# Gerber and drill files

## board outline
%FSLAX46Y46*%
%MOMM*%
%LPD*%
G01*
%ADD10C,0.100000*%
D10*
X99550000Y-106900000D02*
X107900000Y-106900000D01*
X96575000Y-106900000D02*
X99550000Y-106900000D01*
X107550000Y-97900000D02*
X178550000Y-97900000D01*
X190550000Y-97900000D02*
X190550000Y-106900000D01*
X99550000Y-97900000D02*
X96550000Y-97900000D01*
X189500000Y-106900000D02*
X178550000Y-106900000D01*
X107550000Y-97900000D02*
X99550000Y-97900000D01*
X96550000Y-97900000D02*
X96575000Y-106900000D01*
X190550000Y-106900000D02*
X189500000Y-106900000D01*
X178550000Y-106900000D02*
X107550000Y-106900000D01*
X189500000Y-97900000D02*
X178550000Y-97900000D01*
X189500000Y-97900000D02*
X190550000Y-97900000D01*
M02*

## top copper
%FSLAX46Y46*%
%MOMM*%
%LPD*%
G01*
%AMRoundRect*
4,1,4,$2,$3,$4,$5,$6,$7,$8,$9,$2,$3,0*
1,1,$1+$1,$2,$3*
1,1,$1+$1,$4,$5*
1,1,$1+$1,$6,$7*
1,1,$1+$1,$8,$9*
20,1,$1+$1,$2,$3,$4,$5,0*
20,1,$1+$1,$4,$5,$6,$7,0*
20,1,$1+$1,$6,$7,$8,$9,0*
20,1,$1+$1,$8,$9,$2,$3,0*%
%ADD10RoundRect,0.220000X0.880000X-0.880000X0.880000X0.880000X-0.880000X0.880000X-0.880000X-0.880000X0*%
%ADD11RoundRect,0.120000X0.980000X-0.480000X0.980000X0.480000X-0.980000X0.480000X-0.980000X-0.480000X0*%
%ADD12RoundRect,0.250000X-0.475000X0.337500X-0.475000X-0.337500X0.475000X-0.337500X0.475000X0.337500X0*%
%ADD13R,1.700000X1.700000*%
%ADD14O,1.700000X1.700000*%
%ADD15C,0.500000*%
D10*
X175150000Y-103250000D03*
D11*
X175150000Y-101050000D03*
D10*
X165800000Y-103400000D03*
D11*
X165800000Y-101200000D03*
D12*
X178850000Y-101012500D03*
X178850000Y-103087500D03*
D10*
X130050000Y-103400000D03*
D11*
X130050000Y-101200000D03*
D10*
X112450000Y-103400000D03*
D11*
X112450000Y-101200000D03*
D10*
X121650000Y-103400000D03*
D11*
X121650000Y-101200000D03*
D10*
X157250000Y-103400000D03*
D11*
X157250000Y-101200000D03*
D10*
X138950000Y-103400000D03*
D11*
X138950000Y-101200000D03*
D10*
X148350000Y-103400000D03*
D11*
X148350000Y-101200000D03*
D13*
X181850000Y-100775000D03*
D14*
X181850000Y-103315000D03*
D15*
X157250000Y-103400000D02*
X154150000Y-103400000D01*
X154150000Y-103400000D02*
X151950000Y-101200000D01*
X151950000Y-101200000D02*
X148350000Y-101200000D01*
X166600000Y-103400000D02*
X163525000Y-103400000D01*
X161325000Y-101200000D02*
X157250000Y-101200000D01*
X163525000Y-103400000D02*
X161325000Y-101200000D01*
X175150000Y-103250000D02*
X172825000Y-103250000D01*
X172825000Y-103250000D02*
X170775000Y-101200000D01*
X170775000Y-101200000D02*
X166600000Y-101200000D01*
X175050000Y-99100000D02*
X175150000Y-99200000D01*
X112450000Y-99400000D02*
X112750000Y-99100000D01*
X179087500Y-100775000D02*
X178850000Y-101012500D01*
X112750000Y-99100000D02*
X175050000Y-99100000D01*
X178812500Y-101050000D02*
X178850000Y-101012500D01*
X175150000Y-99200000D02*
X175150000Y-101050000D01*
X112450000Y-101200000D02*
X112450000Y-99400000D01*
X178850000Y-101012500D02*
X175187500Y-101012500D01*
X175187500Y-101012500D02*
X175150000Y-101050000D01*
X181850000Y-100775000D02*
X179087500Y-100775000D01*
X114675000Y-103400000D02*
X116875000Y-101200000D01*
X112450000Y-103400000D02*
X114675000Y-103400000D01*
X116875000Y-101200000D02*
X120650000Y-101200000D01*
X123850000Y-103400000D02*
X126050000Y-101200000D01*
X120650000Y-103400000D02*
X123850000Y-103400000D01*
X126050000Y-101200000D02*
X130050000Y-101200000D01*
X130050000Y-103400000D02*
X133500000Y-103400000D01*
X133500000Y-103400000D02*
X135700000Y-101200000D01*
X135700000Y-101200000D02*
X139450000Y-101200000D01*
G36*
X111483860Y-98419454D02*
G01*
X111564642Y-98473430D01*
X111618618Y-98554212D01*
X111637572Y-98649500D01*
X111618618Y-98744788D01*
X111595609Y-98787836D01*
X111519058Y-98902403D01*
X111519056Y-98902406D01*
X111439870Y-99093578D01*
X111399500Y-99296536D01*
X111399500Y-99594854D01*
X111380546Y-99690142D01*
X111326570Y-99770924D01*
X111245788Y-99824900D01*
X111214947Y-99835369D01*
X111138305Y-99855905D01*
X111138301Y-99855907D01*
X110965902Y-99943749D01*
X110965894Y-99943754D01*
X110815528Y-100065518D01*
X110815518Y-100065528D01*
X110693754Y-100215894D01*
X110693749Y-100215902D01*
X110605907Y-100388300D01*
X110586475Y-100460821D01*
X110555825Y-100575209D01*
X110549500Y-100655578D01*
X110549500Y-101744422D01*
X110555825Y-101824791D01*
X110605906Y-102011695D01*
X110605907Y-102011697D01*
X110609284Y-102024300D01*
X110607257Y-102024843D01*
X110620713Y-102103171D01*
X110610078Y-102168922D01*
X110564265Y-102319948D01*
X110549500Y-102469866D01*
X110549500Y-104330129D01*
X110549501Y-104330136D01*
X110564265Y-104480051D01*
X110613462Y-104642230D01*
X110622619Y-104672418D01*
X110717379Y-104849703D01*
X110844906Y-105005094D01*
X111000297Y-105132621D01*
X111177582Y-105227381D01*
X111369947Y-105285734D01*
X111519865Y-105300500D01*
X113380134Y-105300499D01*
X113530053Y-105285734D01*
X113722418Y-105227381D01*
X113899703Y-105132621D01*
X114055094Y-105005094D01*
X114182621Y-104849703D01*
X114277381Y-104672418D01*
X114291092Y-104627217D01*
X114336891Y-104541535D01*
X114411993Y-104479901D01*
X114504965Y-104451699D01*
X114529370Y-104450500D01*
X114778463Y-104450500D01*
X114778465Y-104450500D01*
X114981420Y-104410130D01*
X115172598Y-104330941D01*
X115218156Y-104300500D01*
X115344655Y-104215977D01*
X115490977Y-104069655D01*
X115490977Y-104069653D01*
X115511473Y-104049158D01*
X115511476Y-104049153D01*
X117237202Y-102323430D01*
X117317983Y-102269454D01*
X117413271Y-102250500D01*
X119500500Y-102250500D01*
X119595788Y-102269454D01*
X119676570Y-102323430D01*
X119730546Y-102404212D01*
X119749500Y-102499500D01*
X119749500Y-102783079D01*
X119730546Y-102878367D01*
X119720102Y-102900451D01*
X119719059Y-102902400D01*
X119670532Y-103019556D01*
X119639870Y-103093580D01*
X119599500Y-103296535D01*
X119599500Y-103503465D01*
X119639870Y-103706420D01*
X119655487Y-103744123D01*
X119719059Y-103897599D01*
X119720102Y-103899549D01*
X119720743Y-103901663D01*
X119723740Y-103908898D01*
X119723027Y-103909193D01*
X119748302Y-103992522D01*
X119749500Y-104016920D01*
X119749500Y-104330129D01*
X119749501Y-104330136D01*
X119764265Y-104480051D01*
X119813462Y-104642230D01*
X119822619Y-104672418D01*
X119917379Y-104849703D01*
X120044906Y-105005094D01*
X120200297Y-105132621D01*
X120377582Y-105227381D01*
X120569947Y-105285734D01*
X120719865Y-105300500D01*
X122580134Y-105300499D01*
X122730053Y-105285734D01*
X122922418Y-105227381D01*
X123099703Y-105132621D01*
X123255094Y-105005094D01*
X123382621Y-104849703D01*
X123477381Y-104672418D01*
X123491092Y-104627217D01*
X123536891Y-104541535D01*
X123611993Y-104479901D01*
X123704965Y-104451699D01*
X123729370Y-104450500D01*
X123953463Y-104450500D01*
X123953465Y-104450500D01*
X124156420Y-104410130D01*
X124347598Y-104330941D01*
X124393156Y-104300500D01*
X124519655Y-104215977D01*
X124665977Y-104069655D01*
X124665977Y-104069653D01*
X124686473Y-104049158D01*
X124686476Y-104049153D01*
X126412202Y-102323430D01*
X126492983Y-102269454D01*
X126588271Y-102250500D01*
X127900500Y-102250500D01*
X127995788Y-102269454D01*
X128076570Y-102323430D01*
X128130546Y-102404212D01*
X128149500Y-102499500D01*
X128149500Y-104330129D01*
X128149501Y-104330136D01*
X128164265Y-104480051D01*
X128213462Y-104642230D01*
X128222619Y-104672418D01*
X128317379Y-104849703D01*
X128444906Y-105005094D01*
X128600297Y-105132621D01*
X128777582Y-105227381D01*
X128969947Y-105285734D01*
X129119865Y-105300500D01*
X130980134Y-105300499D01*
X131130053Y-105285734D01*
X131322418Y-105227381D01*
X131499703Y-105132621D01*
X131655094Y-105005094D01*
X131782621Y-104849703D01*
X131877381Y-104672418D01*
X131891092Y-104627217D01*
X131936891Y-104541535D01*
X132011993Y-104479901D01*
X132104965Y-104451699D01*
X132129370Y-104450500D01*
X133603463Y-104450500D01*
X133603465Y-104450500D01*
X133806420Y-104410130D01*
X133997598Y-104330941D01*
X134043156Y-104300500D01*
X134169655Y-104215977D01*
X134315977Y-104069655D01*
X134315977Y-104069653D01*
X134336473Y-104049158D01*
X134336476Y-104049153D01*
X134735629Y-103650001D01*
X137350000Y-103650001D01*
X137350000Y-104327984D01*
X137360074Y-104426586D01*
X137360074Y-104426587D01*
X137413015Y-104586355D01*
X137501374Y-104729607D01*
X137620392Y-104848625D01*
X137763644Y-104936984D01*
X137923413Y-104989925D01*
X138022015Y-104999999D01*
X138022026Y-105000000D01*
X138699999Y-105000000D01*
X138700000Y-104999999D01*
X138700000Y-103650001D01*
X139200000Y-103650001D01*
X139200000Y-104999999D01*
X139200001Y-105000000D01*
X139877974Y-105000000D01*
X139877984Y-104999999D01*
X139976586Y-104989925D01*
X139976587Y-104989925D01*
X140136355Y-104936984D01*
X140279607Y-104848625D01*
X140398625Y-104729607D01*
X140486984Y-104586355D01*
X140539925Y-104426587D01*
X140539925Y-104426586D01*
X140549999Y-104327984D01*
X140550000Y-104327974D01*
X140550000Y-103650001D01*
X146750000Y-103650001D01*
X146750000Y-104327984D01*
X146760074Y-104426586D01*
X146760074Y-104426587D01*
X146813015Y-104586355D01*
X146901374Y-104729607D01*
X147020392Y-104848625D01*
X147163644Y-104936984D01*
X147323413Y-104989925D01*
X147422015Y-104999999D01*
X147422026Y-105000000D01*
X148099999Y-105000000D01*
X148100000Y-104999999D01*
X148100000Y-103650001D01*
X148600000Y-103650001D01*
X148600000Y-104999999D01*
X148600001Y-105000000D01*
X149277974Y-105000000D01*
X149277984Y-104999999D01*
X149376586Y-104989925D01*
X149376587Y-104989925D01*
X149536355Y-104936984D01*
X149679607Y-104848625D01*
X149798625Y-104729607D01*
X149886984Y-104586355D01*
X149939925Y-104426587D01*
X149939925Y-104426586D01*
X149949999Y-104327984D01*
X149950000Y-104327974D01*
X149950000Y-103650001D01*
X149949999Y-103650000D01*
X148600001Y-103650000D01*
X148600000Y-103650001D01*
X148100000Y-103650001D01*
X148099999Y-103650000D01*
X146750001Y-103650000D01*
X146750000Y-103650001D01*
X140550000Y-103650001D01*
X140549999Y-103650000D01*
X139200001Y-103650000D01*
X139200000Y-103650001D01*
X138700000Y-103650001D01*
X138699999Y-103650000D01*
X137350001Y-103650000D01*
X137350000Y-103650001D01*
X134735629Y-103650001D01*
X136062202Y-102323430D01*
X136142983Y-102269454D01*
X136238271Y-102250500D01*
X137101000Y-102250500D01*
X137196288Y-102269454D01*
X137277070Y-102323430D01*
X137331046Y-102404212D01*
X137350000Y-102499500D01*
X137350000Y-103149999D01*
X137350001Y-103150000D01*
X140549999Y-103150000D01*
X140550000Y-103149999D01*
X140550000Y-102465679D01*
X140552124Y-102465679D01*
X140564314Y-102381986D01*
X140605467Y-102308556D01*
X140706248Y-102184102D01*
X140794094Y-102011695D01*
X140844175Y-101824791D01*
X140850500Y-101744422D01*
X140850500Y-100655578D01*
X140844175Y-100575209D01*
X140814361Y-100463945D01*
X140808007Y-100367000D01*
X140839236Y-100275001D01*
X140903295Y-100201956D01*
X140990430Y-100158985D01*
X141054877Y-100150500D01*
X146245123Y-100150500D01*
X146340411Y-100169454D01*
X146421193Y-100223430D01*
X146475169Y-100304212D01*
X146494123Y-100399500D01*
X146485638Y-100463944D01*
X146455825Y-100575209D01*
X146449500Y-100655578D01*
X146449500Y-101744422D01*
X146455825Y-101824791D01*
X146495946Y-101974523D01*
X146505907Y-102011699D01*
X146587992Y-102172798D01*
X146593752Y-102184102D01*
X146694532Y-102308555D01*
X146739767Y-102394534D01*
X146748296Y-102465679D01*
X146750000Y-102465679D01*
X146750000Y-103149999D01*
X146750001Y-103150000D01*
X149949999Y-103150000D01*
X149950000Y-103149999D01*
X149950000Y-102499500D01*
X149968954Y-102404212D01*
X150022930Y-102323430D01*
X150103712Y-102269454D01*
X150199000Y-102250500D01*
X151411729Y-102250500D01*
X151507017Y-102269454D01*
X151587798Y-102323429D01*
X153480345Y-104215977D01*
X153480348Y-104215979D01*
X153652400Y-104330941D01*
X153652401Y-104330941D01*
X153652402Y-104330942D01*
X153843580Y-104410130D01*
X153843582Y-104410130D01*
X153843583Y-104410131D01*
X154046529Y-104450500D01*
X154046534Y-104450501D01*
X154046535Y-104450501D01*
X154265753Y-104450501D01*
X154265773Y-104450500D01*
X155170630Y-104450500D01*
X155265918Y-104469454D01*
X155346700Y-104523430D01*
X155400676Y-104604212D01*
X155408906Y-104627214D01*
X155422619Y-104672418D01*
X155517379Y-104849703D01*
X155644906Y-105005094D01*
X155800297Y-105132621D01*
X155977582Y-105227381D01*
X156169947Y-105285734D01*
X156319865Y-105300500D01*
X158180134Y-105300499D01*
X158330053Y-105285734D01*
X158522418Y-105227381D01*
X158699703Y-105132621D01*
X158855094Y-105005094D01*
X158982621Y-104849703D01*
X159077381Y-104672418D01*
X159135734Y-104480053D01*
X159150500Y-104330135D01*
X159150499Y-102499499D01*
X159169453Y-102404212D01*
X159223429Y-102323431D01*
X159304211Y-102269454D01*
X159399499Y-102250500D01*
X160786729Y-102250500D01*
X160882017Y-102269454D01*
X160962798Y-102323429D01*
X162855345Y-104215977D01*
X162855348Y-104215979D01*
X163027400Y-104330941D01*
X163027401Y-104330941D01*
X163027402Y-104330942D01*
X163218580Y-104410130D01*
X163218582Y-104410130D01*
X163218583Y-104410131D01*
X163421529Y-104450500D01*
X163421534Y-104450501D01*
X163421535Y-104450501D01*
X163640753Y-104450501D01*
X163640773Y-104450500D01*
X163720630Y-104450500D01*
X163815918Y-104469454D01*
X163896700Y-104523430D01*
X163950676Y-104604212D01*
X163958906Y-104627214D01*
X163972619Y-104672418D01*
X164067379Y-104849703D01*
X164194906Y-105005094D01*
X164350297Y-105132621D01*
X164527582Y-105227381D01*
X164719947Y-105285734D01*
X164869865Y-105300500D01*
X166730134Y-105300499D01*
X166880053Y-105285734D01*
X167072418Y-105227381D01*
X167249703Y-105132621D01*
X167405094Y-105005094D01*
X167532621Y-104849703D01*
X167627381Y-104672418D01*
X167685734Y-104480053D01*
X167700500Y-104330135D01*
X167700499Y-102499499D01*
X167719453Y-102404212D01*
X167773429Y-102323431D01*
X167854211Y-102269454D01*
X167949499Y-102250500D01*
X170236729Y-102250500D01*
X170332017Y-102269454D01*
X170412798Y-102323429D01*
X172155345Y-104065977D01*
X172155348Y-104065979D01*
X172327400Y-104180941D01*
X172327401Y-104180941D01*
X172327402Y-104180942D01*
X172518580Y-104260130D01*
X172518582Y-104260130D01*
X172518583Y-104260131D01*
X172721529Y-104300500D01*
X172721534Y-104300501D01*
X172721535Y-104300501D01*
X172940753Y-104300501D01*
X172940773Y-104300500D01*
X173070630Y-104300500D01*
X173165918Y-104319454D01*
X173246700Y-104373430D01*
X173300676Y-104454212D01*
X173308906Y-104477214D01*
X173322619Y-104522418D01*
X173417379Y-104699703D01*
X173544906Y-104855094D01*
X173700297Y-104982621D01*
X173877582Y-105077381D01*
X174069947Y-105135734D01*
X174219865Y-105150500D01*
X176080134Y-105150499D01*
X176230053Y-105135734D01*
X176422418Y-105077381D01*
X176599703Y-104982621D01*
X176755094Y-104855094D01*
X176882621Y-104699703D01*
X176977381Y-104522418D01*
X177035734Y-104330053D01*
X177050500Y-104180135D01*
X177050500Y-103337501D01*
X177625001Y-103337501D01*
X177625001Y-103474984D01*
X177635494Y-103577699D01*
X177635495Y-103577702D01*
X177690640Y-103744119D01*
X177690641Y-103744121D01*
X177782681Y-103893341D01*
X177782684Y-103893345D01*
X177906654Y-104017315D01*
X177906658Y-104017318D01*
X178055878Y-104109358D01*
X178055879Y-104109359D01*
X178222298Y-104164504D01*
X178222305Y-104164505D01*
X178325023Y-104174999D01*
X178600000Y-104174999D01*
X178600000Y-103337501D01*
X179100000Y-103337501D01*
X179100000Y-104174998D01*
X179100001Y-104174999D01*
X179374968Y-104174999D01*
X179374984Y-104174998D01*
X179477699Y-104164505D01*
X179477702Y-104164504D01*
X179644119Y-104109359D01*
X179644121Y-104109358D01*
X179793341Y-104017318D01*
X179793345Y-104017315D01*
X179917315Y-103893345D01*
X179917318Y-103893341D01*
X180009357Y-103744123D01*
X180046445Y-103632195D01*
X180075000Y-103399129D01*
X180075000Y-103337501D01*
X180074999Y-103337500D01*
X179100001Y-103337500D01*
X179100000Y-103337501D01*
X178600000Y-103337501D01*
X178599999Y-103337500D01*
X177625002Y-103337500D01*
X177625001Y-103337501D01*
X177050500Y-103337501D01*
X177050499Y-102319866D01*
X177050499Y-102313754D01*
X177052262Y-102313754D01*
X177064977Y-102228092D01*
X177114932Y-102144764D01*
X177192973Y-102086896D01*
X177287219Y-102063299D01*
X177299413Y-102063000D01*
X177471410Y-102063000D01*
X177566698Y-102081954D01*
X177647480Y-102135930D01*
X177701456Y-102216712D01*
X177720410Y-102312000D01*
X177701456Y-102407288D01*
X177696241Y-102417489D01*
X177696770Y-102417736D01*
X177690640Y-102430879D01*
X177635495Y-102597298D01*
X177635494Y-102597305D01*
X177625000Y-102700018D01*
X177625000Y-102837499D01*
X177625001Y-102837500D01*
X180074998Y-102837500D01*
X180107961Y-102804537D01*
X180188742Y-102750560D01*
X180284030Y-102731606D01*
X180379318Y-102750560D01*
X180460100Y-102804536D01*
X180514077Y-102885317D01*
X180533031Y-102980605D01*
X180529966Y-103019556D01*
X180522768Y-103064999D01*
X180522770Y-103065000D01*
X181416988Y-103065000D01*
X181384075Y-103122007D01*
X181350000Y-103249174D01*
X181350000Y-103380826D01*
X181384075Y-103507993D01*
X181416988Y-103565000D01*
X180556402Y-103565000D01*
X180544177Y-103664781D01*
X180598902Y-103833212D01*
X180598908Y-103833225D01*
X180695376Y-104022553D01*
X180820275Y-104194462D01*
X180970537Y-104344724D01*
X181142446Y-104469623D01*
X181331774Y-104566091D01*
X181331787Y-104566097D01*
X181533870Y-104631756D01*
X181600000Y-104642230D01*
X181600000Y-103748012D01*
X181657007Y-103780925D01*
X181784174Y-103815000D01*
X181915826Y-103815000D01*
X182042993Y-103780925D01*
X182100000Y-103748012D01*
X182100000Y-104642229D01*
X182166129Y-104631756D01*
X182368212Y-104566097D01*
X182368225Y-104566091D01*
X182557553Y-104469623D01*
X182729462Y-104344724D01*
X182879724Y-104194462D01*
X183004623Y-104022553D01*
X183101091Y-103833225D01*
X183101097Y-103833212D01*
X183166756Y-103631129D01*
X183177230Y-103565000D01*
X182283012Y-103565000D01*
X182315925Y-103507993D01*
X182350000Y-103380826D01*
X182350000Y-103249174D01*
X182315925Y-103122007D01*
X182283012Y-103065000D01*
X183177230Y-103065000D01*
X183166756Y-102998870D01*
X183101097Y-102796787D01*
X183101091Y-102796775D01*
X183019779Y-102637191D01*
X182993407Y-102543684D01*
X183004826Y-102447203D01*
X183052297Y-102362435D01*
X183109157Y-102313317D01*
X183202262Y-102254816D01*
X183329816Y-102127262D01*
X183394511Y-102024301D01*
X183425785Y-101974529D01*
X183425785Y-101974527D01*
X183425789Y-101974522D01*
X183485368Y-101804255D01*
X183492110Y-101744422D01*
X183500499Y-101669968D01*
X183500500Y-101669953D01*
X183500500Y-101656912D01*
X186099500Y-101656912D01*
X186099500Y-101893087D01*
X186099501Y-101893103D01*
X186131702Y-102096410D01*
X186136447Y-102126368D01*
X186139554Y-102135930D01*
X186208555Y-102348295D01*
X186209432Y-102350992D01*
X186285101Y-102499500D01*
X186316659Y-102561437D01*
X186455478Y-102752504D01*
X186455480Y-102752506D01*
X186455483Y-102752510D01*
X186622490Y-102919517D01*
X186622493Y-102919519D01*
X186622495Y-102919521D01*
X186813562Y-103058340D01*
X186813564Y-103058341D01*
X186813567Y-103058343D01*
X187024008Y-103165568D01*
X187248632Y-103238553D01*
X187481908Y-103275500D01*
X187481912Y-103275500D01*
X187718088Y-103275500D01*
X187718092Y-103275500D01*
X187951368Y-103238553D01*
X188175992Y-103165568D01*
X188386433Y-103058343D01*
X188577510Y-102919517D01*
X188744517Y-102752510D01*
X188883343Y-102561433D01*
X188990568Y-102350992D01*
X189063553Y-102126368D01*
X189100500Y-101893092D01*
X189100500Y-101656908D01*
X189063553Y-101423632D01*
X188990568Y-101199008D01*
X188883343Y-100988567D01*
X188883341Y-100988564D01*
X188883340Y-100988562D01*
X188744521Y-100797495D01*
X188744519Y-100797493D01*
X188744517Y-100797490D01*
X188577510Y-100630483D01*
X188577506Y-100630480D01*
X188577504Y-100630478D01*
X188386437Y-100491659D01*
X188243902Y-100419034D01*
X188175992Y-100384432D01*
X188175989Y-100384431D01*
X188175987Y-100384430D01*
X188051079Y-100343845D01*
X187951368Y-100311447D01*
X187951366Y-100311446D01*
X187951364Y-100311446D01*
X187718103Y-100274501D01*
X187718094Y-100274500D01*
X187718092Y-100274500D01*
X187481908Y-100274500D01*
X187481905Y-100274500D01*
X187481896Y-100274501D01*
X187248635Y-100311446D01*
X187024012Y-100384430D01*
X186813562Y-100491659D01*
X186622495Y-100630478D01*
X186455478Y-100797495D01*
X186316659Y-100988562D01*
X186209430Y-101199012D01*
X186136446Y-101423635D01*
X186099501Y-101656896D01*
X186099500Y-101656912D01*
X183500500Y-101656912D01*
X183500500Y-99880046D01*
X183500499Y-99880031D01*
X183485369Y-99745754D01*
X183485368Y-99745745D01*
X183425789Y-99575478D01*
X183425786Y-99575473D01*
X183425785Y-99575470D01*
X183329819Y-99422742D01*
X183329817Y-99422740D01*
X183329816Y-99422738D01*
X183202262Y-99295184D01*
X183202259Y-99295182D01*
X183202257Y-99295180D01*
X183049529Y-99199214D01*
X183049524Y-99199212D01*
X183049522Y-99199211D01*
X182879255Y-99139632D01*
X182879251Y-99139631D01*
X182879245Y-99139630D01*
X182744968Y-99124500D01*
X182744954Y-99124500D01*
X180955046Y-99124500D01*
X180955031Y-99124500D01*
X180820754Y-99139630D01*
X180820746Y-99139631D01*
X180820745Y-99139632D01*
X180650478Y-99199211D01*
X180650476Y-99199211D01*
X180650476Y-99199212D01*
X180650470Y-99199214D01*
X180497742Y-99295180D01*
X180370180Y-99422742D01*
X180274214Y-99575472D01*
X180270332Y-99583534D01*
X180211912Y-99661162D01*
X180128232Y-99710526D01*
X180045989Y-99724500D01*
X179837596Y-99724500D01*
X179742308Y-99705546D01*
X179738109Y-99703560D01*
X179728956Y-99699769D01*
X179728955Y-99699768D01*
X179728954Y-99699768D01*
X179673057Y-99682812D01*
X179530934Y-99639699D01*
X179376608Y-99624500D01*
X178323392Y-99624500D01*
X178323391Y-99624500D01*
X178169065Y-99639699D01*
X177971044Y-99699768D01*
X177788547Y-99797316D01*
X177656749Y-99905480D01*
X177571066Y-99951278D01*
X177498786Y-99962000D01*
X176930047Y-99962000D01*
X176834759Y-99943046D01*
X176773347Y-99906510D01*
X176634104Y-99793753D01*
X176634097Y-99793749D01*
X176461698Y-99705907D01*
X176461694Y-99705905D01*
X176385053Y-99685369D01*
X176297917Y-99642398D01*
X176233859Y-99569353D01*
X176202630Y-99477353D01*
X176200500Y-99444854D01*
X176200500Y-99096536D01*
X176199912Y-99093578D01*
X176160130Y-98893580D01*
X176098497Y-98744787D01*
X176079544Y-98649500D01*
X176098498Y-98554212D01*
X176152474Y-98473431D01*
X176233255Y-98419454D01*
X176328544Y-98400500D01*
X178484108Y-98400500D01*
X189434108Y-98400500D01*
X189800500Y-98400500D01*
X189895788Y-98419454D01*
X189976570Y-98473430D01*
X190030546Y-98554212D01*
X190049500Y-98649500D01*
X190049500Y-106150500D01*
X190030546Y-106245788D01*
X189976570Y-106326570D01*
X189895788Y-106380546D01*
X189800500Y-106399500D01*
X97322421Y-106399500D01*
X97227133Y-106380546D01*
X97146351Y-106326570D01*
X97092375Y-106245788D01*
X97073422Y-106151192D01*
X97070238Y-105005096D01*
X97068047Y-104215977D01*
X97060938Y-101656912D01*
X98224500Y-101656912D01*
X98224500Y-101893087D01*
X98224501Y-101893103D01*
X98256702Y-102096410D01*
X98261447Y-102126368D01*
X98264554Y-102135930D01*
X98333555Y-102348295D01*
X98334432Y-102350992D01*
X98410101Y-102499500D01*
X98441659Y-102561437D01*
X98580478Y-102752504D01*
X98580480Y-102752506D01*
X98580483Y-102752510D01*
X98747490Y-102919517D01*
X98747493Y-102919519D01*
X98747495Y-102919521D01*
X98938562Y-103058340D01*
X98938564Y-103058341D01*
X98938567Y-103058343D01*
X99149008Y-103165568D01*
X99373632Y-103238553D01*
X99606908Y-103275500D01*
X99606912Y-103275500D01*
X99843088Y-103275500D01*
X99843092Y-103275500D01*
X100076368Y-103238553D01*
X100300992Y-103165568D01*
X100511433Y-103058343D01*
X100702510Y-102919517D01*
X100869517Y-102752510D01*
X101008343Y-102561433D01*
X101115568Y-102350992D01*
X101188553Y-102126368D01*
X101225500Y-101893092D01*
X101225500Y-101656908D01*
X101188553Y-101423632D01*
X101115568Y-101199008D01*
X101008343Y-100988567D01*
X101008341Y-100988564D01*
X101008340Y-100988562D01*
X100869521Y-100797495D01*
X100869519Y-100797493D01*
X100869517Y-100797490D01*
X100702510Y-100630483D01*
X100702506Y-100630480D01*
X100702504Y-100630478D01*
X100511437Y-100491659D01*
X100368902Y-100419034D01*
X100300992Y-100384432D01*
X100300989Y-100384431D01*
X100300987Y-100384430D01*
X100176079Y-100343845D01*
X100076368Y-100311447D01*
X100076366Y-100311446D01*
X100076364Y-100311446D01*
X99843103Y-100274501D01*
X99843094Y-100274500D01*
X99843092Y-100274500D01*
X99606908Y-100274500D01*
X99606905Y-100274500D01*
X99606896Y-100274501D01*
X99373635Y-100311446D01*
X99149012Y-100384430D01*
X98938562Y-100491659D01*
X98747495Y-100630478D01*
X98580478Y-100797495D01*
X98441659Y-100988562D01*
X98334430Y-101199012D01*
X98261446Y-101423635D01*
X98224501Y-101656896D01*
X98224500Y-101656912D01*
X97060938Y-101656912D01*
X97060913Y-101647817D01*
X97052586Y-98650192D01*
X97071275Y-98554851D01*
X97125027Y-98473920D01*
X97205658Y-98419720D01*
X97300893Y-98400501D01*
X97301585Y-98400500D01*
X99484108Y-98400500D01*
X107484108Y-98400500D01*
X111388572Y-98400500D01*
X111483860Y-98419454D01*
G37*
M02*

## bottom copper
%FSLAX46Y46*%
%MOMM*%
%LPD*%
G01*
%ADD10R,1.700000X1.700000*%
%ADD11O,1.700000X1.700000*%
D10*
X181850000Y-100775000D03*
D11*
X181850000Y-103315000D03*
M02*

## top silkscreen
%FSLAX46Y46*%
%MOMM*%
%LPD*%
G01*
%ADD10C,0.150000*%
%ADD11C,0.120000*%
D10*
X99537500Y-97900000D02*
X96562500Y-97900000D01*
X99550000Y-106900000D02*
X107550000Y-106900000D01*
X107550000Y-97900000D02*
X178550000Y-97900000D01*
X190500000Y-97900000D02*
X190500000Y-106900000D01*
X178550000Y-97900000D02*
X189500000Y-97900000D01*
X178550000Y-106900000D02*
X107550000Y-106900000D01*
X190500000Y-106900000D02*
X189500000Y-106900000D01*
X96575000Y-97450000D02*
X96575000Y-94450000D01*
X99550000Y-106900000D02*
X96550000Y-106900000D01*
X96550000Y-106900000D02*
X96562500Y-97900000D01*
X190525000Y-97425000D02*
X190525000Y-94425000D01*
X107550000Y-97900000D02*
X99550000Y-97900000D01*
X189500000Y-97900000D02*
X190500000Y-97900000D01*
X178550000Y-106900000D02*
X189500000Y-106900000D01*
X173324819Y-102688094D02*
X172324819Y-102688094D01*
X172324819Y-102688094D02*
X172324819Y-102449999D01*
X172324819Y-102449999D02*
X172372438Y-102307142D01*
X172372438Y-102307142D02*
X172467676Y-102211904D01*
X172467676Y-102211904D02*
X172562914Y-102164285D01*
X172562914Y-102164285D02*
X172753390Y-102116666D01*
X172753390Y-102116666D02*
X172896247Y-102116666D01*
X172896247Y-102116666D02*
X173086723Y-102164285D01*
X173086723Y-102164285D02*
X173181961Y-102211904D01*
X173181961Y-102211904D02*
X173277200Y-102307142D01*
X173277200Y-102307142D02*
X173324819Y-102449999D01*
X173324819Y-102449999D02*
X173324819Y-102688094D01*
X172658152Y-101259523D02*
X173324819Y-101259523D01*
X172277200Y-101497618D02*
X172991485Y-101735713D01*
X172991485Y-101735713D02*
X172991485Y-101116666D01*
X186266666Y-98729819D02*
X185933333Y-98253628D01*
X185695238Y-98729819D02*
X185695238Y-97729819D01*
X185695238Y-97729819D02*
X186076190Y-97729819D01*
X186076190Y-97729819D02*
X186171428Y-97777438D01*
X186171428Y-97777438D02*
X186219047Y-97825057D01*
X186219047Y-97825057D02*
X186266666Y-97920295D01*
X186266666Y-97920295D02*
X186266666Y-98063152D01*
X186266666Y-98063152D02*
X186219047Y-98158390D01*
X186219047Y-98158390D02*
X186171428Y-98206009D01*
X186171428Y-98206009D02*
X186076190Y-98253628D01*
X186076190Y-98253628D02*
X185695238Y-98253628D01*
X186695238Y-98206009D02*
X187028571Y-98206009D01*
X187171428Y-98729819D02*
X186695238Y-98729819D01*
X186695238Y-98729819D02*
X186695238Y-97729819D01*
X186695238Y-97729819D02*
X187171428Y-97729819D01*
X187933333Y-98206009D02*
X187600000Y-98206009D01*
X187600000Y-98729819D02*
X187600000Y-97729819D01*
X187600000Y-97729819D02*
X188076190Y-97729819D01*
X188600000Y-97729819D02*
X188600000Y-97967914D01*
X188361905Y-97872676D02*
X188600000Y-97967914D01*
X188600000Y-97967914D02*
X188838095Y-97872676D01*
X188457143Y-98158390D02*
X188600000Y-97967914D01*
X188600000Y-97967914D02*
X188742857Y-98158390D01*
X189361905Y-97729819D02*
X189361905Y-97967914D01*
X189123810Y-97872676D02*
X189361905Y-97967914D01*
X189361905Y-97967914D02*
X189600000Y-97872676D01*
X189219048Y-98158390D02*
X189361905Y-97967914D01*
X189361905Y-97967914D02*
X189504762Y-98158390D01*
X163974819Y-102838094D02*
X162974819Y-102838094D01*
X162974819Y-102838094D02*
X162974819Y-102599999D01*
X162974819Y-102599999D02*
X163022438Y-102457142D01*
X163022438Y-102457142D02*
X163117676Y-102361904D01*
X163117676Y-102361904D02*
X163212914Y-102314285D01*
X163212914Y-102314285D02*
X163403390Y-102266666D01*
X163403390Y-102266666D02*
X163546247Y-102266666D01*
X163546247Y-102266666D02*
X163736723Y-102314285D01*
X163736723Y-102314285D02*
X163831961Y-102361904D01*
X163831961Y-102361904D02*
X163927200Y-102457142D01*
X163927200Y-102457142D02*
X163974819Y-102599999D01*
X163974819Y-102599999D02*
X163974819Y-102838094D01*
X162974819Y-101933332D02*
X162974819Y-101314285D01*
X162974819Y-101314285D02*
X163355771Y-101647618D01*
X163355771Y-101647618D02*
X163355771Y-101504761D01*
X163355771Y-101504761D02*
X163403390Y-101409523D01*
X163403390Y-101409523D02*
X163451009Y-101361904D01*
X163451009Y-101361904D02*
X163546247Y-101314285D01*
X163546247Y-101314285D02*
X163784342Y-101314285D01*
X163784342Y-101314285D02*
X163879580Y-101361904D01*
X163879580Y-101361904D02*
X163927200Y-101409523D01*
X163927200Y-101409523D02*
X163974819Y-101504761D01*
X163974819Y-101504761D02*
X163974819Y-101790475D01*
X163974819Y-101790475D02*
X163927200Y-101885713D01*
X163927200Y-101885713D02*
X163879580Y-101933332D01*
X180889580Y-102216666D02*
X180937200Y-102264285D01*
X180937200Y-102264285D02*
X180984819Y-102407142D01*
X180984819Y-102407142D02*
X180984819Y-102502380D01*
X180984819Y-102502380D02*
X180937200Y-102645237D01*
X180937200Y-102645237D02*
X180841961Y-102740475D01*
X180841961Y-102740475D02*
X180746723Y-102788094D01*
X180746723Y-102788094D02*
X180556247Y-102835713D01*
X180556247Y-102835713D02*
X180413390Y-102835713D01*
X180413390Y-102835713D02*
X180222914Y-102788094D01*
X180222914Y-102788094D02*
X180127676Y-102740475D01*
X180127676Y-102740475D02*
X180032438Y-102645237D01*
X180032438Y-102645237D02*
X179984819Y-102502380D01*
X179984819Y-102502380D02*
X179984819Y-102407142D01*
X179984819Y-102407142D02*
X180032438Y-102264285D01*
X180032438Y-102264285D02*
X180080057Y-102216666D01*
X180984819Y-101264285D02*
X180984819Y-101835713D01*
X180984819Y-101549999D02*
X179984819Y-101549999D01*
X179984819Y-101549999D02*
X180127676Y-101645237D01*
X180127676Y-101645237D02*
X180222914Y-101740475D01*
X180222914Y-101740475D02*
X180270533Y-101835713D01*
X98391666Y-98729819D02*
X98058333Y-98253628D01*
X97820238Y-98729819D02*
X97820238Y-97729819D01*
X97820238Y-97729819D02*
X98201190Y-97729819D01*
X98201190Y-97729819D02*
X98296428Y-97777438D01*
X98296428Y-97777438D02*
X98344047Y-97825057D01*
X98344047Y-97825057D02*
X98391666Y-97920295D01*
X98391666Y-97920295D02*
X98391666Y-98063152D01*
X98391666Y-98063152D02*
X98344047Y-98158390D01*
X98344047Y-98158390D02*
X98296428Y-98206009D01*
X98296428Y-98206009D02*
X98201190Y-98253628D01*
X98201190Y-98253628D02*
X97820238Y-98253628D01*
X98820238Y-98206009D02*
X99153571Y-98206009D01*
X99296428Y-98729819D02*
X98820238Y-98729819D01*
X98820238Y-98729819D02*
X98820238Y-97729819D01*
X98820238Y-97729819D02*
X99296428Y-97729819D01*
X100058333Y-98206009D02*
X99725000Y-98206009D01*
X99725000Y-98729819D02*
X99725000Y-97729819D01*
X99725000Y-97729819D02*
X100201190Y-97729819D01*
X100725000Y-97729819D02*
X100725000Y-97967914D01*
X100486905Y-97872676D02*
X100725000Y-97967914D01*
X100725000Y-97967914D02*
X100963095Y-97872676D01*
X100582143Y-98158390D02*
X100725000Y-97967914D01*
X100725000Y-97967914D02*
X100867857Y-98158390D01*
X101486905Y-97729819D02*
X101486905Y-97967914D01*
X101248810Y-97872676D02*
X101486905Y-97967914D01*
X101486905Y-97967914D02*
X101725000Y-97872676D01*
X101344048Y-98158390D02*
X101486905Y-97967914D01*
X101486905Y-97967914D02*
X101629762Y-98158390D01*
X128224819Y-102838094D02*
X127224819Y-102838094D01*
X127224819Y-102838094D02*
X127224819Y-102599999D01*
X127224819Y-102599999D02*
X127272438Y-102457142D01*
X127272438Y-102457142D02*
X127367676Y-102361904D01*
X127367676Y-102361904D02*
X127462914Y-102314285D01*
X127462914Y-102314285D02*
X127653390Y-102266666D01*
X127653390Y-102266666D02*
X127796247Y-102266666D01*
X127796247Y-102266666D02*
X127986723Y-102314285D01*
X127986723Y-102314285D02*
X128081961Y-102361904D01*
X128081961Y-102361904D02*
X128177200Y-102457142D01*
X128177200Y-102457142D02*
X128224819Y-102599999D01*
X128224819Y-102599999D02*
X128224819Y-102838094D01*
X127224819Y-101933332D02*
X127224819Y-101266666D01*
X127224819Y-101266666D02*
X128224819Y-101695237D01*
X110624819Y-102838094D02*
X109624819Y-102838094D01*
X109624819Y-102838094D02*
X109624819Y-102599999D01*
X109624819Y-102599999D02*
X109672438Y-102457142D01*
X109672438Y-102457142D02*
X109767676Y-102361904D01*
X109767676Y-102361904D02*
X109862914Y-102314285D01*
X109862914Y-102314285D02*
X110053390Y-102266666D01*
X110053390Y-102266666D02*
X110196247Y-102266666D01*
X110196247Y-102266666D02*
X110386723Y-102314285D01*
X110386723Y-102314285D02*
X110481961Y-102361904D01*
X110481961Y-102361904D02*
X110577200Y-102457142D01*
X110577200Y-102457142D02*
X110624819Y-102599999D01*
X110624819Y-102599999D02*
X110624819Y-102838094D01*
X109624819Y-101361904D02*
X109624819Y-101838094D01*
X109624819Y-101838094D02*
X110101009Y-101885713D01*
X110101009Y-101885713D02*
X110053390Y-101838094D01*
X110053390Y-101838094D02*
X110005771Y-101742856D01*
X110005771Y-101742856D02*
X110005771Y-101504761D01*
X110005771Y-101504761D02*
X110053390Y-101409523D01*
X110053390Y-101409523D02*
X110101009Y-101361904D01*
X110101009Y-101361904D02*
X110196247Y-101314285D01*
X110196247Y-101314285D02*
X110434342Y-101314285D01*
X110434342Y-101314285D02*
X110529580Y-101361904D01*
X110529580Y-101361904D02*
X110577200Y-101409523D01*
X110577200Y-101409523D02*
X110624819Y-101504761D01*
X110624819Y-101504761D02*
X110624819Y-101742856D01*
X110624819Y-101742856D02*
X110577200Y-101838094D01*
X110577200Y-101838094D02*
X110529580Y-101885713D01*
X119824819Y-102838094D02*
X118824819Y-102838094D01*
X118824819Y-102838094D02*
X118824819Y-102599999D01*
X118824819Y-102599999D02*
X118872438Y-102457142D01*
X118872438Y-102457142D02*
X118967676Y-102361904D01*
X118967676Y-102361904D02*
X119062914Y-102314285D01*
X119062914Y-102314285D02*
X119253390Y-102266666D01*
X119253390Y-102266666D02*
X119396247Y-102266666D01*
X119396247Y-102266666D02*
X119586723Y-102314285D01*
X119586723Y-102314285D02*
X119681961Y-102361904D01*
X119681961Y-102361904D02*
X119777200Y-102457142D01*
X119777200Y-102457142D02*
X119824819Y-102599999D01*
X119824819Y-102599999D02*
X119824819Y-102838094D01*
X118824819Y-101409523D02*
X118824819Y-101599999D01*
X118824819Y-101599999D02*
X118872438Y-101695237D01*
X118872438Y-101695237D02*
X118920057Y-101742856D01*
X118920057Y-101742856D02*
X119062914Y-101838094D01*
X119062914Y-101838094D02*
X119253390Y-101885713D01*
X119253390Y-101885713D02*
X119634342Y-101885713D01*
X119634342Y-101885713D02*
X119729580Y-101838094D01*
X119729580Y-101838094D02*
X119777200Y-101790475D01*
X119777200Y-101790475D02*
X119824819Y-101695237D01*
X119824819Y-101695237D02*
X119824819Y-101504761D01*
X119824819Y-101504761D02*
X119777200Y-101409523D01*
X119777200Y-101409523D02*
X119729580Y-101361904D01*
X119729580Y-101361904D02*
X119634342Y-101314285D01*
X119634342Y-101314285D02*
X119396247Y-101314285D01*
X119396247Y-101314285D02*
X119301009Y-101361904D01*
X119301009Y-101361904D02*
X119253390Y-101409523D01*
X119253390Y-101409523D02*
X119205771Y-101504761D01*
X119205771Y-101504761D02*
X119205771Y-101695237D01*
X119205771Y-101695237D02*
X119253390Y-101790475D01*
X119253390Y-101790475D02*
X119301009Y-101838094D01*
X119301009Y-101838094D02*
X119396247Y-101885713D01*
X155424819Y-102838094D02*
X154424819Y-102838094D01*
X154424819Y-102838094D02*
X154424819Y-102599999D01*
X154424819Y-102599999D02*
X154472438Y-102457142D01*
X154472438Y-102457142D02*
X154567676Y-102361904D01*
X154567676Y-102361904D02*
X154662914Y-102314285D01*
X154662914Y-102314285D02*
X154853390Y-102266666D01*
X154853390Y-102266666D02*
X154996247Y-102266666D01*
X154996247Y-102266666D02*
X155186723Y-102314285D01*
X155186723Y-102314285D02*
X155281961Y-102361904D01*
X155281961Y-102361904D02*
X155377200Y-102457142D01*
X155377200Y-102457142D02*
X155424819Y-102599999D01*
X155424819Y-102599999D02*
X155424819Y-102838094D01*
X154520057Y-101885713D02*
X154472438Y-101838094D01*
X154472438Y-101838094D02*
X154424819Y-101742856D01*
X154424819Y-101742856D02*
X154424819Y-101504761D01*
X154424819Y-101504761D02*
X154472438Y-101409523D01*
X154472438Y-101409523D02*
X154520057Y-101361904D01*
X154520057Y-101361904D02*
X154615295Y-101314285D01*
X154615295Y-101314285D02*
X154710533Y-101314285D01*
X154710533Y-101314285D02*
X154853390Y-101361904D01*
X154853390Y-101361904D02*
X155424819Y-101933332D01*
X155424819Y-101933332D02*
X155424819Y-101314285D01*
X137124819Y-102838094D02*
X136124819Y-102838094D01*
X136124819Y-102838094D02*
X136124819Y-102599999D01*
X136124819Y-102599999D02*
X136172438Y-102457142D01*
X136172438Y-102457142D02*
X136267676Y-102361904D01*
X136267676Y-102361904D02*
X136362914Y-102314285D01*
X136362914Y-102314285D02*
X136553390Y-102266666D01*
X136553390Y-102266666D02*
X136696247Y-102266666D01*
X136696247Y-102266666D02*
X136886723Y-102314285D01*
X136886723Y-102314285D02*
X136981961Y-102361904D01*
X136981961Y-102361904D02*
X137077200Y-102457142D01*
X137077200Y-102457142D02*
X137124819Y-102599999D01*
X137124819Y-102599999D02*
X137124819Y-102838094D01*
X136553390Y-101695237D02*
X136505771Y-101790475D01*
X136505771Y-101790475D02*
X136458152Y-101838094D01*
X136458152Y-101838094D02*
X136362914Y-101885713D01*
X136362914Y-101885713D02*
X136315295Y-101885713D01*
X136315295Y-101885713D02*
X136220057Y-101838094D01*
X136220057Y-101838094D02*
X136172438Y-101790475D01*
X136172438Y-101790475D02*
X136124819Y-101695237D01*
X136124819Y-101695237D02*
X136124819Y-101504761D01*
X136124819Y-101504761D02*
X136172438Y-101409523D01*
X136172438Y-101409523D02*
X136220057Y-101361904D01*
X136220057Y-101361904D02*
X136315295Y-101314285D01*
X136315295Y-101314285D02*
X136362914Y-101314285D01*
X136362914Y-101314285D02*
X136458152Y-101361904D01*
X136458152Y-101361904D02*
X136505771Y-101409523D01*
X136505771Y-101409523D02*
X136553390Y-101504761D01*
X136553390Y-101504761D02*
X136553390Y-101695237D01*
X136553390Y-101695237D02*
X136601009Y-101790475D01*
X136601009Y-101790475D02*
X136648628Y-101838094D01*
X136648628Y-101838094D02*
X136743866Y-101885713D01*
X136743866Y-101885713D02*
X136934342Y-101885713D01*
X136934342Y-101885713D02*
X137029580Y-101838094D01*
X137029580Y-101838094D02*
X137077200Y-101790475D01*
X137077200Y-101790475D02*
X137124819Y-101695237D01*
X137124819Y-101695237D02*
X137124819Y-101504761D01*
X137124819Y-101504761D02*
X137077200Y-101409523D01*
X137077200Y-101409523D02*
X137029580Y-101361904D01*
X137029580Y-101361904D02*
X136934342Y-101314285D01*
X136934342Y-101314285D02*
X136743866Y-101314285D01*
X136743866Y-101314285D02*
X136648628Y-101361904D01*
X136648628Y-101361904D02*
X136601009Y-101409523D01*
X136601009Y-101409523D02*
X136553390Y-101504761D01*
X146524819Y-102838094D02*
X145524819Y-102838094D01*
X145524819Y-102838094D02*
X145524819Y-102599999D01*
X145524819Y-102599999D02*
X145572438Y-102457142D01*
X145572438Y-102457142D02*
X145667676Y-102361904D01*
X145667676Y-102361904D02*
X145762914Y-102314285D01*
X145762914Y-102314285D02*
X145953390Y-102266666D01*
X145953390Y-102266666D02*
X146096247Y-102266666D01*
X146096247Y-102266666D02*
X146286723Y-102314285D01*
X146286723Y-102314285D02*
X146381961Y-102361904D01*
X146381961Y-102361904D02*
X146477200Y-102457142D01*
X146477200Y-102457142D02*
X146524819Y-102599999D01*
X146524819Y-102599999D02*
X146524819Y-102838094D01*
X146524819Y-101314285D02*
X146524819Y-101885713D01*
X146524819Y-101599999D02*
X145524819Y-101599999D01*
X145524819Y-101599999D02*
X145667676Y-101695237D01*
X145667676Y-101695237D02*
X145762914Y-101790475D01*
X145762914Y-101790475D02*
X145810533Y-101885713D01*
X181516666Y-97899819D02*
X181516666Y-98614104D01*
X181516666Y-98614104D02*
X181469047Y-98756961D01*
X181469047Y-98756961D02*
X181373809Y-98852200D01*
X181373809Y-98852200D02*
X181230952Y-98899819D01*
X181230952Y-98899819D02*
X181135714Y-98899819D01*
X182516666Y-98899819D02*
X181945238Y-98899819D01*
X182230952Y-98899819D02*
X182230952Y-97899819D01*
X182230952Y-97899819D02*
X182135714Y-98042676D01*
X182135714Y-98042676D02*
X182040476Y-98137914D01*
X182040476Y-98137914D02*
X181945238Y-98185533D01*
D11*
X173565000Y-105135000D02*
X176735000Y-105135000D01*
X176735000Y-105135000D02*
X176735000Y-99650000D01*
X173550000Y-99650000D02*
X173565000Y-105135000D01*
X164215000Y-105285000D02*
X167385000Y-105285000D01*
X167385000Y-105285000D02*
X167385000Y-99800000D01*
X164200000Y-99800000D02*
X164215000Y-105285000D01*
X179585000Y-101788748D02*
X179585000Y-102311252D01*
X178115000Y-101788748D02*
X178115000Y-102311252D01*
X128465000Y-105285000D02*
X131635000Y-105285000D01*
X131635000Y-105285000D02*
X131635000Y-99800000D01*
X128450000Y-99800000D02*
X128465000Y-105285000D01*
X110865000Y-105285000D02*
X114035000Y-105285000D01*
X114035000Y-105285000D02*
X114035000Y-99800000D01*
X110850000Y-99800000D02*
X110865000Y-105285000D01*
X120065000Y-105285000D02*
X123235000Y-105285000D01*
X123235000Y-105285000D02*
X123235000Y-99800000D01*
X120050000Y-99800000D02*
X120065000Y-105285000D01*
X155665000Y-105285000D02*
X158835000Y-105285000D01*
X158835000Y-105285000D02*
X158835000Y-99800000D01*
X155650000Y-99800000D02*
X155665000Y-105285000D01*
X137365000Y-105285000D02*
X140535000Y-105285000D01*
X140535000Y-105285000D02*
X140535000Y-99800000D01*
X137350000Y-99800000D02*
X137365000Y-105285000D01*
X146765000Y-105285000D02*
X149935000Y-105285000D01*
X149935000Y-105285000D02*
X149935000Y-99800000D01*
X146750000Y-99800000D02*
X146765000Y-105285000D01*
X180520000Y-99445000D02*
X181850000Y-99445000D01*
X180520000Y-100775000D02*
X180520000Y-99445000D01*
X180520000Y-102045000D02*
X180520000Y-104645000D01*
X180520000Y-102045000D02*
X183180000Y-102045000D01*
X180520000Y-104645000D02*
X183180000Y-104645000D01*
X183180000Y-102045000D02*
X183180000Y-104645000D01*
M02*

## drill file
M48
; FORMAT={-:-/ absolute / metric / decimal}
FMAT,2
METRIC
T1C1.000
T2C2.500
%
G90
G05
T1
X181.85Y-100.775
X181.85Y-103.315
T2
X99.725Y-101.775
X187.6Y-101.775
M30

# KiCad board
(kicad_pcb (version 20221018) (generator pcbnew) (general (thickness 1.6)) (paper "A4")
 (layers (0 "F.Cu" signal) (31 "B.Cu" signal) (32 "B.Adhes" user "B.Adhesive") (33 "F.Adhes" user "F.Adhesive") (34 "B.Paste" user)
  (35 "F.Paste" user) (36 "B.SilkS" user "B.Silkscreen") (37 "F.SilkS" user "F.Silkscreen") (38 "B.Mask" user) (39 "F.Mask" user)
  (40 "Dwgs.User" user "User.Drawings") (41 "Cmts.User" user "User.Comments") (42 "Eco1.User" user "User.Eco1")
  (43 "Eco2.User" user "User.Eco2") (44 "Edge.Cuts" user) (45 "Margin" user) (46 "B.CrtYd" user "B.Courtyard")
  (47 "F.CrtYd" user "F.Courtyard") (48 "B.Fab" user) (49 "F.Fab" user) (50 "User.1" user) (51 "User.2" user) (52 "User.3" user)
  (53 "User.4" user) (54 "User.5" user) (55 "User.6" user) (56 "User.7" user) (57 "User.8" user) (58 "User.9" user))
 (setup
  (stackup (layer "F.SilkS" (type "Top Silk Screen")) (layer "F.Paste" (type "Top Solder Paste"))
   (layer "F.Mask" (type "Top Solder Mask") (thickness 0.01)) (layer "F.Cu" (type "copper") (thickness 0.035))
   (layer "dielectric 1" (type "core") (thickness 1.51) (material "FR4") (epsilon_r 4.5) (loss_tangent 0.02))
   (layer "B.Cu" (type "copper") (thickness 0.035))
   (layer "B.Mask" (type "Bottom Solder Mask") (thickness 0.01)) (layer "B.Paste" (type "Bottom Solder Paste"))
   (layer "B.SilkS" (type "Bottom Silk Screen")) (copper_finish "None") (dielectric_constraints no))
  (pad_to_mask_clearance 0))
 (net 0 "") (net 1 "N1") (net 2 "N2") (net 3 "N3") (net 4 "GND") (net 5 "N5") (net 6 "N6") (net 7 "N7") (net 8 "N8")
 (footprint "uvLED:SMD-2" (layer "F.Cu") (at 175.15 101.95 90)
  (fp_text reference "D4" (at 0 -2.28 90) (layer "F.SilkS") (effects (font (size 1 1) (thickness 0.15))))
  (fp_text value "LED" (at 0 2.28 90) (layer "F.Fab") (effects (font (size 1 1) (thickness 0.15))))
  (fp_line (start -3.185 -1.585) (end -3.185 1.585) (stroke (width 0.12) (type solid)) (layer "F.SilkS"))
  (fp_line (start -3.185 1.585) (end 2.3 1.585) (stroke (width 0.12) (type solid)) (layer "F.SilkS"))
  (fp_line (start 2.3 -1.6) (end -3.185 -1.585) (stroke (width 0.12) (type solid)) (layer "F.SilkS"))
  (pad "1" smd roundrect (at -1.3 0 90) (size 2.2 2.2) (layers "F.Cu" "F.Paste" "F.Mask") (roundrect_rratio 0.1) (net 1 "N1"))
  (pad "2" smd roundrect (at 0.9 0 90) (size 1.2 2.2) (layers "F.Cu" "F.Paste" "F.Mask") (roundrect_rratio 0.1) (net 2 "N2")))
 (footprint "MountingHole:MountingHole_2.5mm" (layer "F.Cu") (at 187.6 101.775)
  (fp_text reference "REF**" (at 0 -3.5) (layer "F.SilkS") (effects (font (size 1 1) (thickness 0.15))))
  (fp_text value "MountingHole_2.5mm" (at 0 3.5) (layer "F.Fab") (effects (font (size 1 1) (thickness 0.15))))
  (pad "" np_thru_hole circle (at 0 0) (size 2.5 2.5) (drill 2.5) (layers "*.Cu" "*.Mask")))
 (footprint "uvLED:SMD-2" (layer "F.Cu") (at 165.8 102.1 90)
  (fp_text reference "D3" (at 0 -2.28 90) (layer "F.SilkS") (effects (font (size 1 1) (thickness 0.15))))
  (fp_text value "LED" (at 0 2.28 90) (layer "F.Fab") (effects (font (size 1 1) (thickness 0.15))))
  (fp_line (start -3.185 -1.585) (end -3.185 1.585) (stroke (width 0.12) (type solid)) (layer "F.SilkS"))
  (fp_line (start -3.185 1.585) (end 2.3 1.585) (stroke (width 0.12) (type solid)) (layer "F.SilkS"))
  (fp_line (start 2.3 -1.6) (end -3.185 -1.585) (stroke (width 0.12) (type solid)) (layer "F.SilkS"))
  (pad "1" smd roundrect (at -1.3 0 90) (size 2.2 2.2) (layers "F.Cu" "F.Paste" "F.Mask") (roundrect_rratio 0.1) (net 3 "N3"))
  (pad "2" smd roundrect (at 0.9 0 90) (size 1.2 2.2) (layers "F.Cu" "F.Paste" "F.Mask") (roundrect_rratio 0.1) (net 1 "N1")))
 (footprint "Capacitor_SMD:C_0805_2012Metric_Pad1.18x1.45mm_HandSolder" (layer "F.Cu") (at 178.85 102.05 -90)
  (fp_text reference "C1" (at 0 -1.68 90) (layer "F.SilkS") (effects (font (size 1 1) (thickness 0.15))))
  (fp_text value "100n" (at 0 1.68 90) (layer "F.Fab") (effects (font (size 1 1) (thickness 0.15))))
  (fp_line (start -0.261252 -0.735) (end 0.261252 -0.735) (stroke (width 0.12) (type solid)) (layer "F.SilkS"))
  (fp_line (start -0.261252 0.735) (end 0.261252 0.735) (stroke (width 0.12) (type solid)) (layer "F.SilkS"))
  (pad "1" smd roundrect (at -1.0375 0 270) (size 1.175 1.45) (layers "F.Cu" "F.Paste" "F.Mask") (roundrect_rratio 0.212766) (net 2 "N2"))
  (pad "2" smd roundrect (at 1.0375 0 270) (size 1.175 1.45) (layers "F.Cu" "F.Paste" "F.Mask") (roundrect_rratio 0.212766) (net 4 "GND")))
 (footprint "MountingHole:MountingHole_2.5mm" (layer "F.Cu") (at 99.725 101.775)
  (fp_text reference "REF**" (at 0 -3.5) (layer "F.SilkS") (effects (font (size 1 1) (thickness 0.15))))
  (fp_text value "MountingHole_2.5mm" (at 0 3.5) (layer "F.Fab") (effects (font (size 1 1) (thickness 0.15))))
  (pad "" np_thru_hole circle (at 0 0) (size 2.5 2.5) (drill 2.5) (layers "*.Cu" "*.Mask")))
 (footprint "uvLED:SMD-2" (layer "F.Cu") (at 130.05 102.1 90)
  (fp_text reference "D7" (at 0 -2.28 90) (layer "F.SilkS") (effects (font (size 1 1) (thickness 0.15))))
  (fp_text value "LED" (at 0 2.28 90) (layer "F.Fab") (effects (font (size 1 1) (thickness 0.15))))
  (fp_line (start -3.185 -1.585) (end -3.185 1.585) (stroke (width 0.12) (type solid)) (layer "F.SilkS"))
  (fp_line (start -3.185 1.585) (end 2.3 1.585) (stroke (width 0.12) (type solid)) (layer "F.SilkS"))
  (fp_line (start 2.3 -1.6) (end -3.185 -1.585) (stroke (width 0.12) (type solid)) (layer "F.SilkS"))
  (pad "1" smd roundrect (at -1.3 0 90) (size 2.2 2.2) (layers "F.Cu" "F.Paste" "F.Mask") (roundrect_rratio 0.1) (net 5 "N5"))
  (pad "2" smd roundrect (at 0.9 0 90) (size 1.2 2.2) (layers "F.Cu" "F.Paste" "F.Mask") (roundrect_rratio 0.1) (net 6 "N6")))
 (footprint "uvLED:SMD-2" (layer "F.Cu") (at 112.45 102.1 90)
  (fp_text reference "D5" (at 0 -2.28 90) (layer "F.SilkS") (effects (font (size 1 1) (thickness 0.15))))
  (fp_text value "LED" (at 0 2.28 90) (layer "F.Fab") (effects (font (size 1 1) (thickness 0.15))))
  (fp_line (start -3.185 -1.585) (end -3.185 1.585) (stroke (width 0.12) (type solid)) (layer "F.SilkS"))
  (fp_line (start -3.185 1.585) (end 2.3 1.585) (stroke (width 0.12) (type solid)) (layer "F.SilkS"))
  (fp_line (start 2.3 -1.6) (end -3.185 -1.585) (stroke (width 0.12) (type solid)) (layer "F.SilkS"))
  (pad "1" smd roundrect (at -1.3 0 90) (size 2.2 2.2) (layers "F.Cu" "F.Paste" "F.Mask") (roundrect_rratio 0.1) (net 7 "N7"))
  (pad "2" smd roundrect (at 0.9 0 90) (size 1.2 2.2) (layers "F.Cu" "F.Paste" "F.Mask") (roundrect_rratio 0.1) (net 2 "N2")))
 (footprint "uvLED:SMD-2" (layer "F.Cu") (at 121.65 102.1 90)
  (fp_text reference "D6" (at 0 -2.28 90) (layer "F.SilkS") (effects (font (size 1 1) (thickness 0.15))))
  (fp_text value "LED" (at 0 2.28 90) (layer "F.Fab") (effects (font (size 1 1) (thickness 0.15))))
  (fp_line (start -3.185 -1.585) (end -3.185 1.585) (stroke (width 0.12) (type solid)) (layer "F.SilkS"))
  (fp_line (start -3.185 1.585) (end 2.3 1.585) (stroke (width 0.12) (type solid)) (layer "F.SilkS"))
  (fp_line (start 2.3 -1.6) (end -3.185 -1.585) (stroke (width 0.12) (type solid)) (layer "F.SilkS"))
  (pad "1" smd roundrect (at -1.3 0 90) (size 2.2 2.2) (layers "F.Cu" "F.Paste" "F.Mask") (roundrect_rratio 0.1) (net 6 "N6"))
  (pad "2" smd roundrect (at 0.9 0 90) (size 1.2 2.2) (layers "F.Cu" "F.Paste" "F.Mask") (roundrect_rratio 0.1) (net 7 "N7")))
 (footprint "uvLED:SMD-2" (layer "F.Cu") (at 157.25 102.1 90)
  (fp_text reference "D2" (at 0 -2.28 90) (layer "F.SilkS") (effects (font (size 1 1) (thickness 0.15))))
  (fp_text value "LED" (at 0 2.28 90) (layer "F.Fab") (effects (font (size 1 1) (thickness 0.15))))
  (fp_line (start -3.185 -1.585) (end -3.185 1.585) (stroke (width 0.12) (type solid)) (layer "F.SilkS"))
  (fp_line (start -3.185 1.585) (end 2.3 1.585) (stroke (width 0.12) (type solid)) (layer "F.SilkS"))
  (fp_line (start 2.3 -1.6) (end -3.185 -1.585) (stroke (width 0.12) (type solid)) (layer "F.SilkS"))
  (pad "1" smd roundrect (at -1.3 0 90) (size 2.2 2.2) (layers "F.Cu" "F.Paste" "F.Mask") (roundrect_rratio 0.1) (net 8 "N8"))
  (pad "2" smd roundrect (at 0.9 0 90) (size 1.2 2.2) (layers "F.Cu" "F.Paste" "F.Mask") (roundrect_rratio 0.1) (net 3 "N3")))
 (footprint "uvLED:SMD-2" (layer "F.Cu") (at 138.95 102.1 90)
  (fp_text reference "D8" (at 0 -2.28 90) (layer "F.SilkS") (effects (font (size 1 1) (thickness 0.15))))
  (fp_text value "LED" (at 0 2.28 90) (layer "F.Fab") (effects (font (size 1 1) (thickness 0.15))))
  (fp_line (start -3.185 -1.585) (end -3.185 1.585) (stroke (width 0.12) (type solid)) (layer "F.SilkS"))
  (fp_line (start -3.185 1.585) (end 2.3 1.585) (stroke (width 0.12) (type solid)) (layer "F.SilkS"))
  (fp_line (start 2.3 -1.6) (end -3.185 -1.585) (stroke (width 0.12) (type solid)) (layer "F.SilkS"))
  (pad "1" smd roundrect (at -1.3 0 90) (size 2.2 2.2) (layers "F.Cu" "F.Paste" "F.Mask") (roundrect_rratio 0.1) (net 4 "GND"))
  (pad "2" smd roundrect (at 0.9 0 90) (size 1.2 2.2) (layers "F.Cu" "F.Paste" "F.Mask") (roundrect_rratio 0.1) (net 5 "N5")))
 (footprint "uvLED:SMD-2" (layer "F.Cu") (at 148.35 102.1 90)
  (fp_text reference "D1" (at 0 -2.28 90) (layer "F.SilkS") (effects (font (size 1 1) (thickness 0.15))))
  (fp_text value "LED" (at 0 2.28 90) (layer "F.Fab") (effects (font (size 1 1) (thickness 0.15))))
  (fp_line (start -3.185 -1.585) (end -3.185 1.585) (stroke (width 0.12) (type solid)) (layer "F.SilkS"))
  (fp_line (start -3.185 1.585) (end 2.3 1.585) (stroke (width 0.12) (type solid)) (layer "F.SilkS"))
  (fp_line (start 2.3 -1.6) (end -3.185 -1.585) (stroke (width 0.12) (type solid)) (layer "F.SilkS"))
  (pad "1" smd roundrect (at -1.3 0 90) (size 2.2 2.2) (layers "F.Cu" "F.Paste" "F.Mask") (roundrect_rratio 0.1) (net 4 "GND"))
  (pad "2" smd roundrect (at 0.9 0 90) (size 1.2 2.2) (layers "F.Cu" "F.Paste" "F.Mask") (roundrect_rratio 0.1) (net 8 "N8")))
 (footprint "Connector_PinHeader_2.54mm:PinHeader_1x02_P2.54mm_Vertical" (layer "F.Cu") (at 181.85 100.775)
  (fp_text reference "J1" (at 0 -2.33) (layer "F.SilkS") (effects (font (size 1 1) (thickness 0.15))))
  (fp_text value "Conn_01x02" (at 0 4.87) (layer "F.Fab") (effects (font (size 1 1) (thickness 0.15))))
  (fp_line (start -1.33 -1.33) (end 0 -1.33) (stroke (width 0.12) (type solid)) (layer "F.SilkS"))
  (fp_line (start -1.33 0) (end -1.33 -1.33) (stroke (width 0.12) (type solid)) (layer "F.SilkS"))
  (fp_line (start -1.33 1.27) (end -1.33 3.87) (stroke (width 0.12) (type solid)) (layer "F.SilkS"))
  (fp_line (start -1.33 1.27) (end 1.33 1.27) (stroke (width 0.12) (type solid)) (layer "F.SilkS"))
  (fp_line (start -1.33 3.87) (end 1.33 3.87) (stroke (width 0.12) (type solid)) (layer "F.SilkS"))
  (fp_line (start 1.33 1.27) (end 1.33 3.87) (stroke (width 0.12) (type solid)) (layer "F.SilkS"))
  (pad "1" thru_hole rect (at 0 0) (size 1.7 1.7) (drill 1) (layers "*.Cu" "*.Mask") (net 2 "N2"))
  (pad "2" thru_hole oval (at 0 2.54) (size 1.7 1.7) (drill 1) (layers "*.Cu" "*.Mask") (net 4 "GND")))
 (gr_line (start 99.5375 97.9) (end 96.5625 97.9) (stroke (width 0.15) (type default)) (layer "F.SilkS"))
 (gr_line (start 99.55 106.9) (end 107.55 106.9) (stroke (width 0.15) (type default)) (layer "F.SilkS"))
 (gr_line (start 107.55 97.9) (end 178.55 97.9) (stroke (width 0.15) (type default)) (layer "F.SilkS"))
 (gr_line (start 190.5 97.9) (end 190.5 106.9) (stroke (width 0.15) (type default)) (layer "F.SilkS"))
 (gr_line (start 178.55 97.9) (end 189.5 97.9) (stroke (width 0.15) (type default)) (layer "F.SilkS"))
 (gr_line (start 178.55 106.9) (end 107.55 106.9) (stroke (width 0.15) (type default)) (layer "F.SilkS"))
 (gr_line (start 190.5 106.9) (end 189.5 106.9) (stroke (width 0.15) (type default)) (layer "F.SilkS"))
 (gr_line (start 96.575 97.45) (end 96.575 94.45) (stroke (width 0.15) (type default)) (layer "F.SilkS"))
 (gr_line (start 99.55 106.9) (end 96.55 106.9) (stroke (width 0.15) (type default)) (layer "F.SilkS"))
 (gr_line (start 96.55 106.9) (end 96.5625 97.9) (stroke (width 0.15) (type default)) (layer "F.SilkS"))
 (gr_line (start 190.525 97.425) (end 190.525 94.425) (stroke (width 0.15) (type default)) (layer "F.SilkS"))
 (gr_line (start 107.55 97.9) (end 99.55 97.9) (stroke (width 0.15) (type default)) (layer "F.SilkS"))
 (gr_line (start 189.5 97.9) (end 190.5 97.9) (stroke (width 0.15) (type default)) (layer "F.SilkS"))
 (gr_line (start 178.55 106.9) (end 189.5 106.9) (stroke (width 0.15) (type default)) (layer "F.SilkS"))
 (gr_line (start 99.55 106.9) (end 107.9 106.9) (stroke (width 0.1) (type default)) (layer "Edge.Cuts"))
 (gr_line (start 96.575 106.9) (end 99.55 106.9) (stroke (width 0.1) (type default)) (layer "Edge.Cuts"))
 (gr_line (start 107.55 97.9) (end 178.55 97.9) (stroke (width 0.1) (type default)) (layer "Edge.Cuts"))
 (gr_line (start 190.55 97.9) (end 190.55 106.9) (stroke (width 0.1) (type default)) (layer "Edge.Cuts"))
 (gr_line (start 99.55 97.9) (end 96.55 97.9) (stroke (width 0.1) (type default)) (layer "Edge.Cuts"))
 (gr_line (start 189.5 106.9) (end 178.55 106.9) (stroke (width 0.1) (type default)) (layer "Edge.Cuts"))
 (gr_line (start 107.55 97.9) (end 99.55 97.9) (stroke (width 0.1) (type default)) (layer "Edge.Cuts"))
 (gr_line (start 96.55 97.9) (end 96.575 106.9) (stroke (width 0.1) (type default)) (layer "Edge.Cuts"))
 (gr_line (start 190.55 106.9) (end 189.5 106.9) (stroke (width 0.1) (type default)) (layer "Edge.Cuts"))
 (gr_line (start 178.55 106.9) (end 107.55 106.9) (stroke (width 0.1) (type default)) (layer "Edge.Cuts"))
 (gr_line (start 189.5 97.9) (end 178.55 97.9) (stroke (width 0.1) (type default)) (layer "Edge.Cuts"))
 (gr_line (start 189.5 97.9) (end 190.55 97.9) (stroke (width 0.1) (type default)) (layer "Edge.Cuts"))
 (segment (start 157.25 103.4) (end 154.15 103.4) (width 0.5) (layer "F.Cu") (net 8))
 (segment (start 154.15 103.4) (end 151.95 101.2) (width 0.5) (layer "F.Cu") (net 8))
 (segment (start 151.95 101.2) (end 148.35 101.2) (width 0.5) (layer "F.Cu") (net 8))
 (segment (start 166.6 103.4) (end 163.525 103.4) (width 0.5) (layer "F.Cu") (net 3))
 (segment (start 161.325 101.2) (end 157.25 101.2) (width 0.5) (layer "F.Cu") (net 3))
 (segment (start 163.525 103.4) (end 161.325 101.2) (width 0.5) (layer "F.Cu") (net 3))
 (segment (start 175.15 103.25) (end 172.825 103.25) (width 0.5) (layer "F.Cu") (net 1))
 (segment (start 172.825 103.25) (end 170.775 101.2) (width 0.5) (layer "F.Cu") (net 1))
 (segment (start 170.775 101.2) (end 166.6 101.2) (width 0.5) (layer "F.Cu") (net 1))
 (segment (start 175.05 99.1) (end 175.15 99.2) (width 0.5) (layer "F.Cu") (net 2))
 (segment (start 112.45 99.4) (end 112.75 99.1) (width 0.5) (layer "F.Cu") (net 2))
 (segment (start 179.0875 100.775) (end 178.85 101.0125) (width 0.5) (layer "F.Cu") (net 2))
 (segment (start 112.75 99.1) (end 175.05 99.1) (width 0.5) (layer "F.Cu") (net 2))
 (segment (start 178.8125 101.05) (end 178.85 101.0125) (width 0.5) (layer "F.Cu") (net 2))
 (segment (start 175.15 99.2) (end 175.15 101.05) (width 0.5) (layer "F.Cu") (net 2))
 (segment (start 112.45 101.2) (end 112.45 99.4) (width 0.5) (layer "F.Cu") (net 2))
 (segment (start 178.85 101.0125) (end 175.1875 101.0125) (width 0.5) (layer "F.Cu") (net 2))
 (segment (start 175.1875 101.0125) (end 175.15 101.05) (width 0.5) (layer "F.Cu") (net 2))
 (segment (start 181.85 100.775) (end 179.0875 100.775) (width 0.5) (layer "F.Cu") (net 2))
 (segment (start 114.675 103.4) (end 116.875 101.2) (width 0.5) (layer "F.Cu") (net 7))
 (segment (start 112.45 103.4) (end 114.675 103.4) (width 0.5) (layer "F.Cu") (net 7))
 (segment (start 116.875 101.2) (end 120.65 101.2) (width 0.5) (layer "F.Cu") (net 7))
 (segment (start 123.85 103.4) (end 126.05 101.2) (width 0.5) (layer "F.Cu") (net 6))
 (segment (start 120.65 103.4) (end 123.85 103.4) (width 0.5) (layer "F.Cu") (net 6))
 (segment (start 126.05 101.2) (end 130.05 101.2) (width 0.5) (layer "F.Cu") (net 6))
 (segment (start 130.05 103.4) (end 133.5 103.4) (width 0.5) (layer "F.Cu") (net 5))
 (segment (start 133.5 103.4) (end 135.7 101.2) (width 0.5) (layer "F.Cu") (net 5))
 (segment (start 135.7 101.2) (end 139.45 101.2) (width 0.5) (layer "F.Cu") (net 5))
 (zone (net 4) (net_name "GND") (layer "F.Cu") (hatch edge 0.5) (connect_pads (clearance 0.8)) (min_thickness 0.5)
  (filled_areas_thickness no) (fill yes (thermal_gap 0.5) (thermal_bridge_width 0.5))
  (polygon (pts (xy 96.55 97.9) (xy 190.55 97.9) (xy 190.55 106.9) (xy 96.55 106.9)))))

